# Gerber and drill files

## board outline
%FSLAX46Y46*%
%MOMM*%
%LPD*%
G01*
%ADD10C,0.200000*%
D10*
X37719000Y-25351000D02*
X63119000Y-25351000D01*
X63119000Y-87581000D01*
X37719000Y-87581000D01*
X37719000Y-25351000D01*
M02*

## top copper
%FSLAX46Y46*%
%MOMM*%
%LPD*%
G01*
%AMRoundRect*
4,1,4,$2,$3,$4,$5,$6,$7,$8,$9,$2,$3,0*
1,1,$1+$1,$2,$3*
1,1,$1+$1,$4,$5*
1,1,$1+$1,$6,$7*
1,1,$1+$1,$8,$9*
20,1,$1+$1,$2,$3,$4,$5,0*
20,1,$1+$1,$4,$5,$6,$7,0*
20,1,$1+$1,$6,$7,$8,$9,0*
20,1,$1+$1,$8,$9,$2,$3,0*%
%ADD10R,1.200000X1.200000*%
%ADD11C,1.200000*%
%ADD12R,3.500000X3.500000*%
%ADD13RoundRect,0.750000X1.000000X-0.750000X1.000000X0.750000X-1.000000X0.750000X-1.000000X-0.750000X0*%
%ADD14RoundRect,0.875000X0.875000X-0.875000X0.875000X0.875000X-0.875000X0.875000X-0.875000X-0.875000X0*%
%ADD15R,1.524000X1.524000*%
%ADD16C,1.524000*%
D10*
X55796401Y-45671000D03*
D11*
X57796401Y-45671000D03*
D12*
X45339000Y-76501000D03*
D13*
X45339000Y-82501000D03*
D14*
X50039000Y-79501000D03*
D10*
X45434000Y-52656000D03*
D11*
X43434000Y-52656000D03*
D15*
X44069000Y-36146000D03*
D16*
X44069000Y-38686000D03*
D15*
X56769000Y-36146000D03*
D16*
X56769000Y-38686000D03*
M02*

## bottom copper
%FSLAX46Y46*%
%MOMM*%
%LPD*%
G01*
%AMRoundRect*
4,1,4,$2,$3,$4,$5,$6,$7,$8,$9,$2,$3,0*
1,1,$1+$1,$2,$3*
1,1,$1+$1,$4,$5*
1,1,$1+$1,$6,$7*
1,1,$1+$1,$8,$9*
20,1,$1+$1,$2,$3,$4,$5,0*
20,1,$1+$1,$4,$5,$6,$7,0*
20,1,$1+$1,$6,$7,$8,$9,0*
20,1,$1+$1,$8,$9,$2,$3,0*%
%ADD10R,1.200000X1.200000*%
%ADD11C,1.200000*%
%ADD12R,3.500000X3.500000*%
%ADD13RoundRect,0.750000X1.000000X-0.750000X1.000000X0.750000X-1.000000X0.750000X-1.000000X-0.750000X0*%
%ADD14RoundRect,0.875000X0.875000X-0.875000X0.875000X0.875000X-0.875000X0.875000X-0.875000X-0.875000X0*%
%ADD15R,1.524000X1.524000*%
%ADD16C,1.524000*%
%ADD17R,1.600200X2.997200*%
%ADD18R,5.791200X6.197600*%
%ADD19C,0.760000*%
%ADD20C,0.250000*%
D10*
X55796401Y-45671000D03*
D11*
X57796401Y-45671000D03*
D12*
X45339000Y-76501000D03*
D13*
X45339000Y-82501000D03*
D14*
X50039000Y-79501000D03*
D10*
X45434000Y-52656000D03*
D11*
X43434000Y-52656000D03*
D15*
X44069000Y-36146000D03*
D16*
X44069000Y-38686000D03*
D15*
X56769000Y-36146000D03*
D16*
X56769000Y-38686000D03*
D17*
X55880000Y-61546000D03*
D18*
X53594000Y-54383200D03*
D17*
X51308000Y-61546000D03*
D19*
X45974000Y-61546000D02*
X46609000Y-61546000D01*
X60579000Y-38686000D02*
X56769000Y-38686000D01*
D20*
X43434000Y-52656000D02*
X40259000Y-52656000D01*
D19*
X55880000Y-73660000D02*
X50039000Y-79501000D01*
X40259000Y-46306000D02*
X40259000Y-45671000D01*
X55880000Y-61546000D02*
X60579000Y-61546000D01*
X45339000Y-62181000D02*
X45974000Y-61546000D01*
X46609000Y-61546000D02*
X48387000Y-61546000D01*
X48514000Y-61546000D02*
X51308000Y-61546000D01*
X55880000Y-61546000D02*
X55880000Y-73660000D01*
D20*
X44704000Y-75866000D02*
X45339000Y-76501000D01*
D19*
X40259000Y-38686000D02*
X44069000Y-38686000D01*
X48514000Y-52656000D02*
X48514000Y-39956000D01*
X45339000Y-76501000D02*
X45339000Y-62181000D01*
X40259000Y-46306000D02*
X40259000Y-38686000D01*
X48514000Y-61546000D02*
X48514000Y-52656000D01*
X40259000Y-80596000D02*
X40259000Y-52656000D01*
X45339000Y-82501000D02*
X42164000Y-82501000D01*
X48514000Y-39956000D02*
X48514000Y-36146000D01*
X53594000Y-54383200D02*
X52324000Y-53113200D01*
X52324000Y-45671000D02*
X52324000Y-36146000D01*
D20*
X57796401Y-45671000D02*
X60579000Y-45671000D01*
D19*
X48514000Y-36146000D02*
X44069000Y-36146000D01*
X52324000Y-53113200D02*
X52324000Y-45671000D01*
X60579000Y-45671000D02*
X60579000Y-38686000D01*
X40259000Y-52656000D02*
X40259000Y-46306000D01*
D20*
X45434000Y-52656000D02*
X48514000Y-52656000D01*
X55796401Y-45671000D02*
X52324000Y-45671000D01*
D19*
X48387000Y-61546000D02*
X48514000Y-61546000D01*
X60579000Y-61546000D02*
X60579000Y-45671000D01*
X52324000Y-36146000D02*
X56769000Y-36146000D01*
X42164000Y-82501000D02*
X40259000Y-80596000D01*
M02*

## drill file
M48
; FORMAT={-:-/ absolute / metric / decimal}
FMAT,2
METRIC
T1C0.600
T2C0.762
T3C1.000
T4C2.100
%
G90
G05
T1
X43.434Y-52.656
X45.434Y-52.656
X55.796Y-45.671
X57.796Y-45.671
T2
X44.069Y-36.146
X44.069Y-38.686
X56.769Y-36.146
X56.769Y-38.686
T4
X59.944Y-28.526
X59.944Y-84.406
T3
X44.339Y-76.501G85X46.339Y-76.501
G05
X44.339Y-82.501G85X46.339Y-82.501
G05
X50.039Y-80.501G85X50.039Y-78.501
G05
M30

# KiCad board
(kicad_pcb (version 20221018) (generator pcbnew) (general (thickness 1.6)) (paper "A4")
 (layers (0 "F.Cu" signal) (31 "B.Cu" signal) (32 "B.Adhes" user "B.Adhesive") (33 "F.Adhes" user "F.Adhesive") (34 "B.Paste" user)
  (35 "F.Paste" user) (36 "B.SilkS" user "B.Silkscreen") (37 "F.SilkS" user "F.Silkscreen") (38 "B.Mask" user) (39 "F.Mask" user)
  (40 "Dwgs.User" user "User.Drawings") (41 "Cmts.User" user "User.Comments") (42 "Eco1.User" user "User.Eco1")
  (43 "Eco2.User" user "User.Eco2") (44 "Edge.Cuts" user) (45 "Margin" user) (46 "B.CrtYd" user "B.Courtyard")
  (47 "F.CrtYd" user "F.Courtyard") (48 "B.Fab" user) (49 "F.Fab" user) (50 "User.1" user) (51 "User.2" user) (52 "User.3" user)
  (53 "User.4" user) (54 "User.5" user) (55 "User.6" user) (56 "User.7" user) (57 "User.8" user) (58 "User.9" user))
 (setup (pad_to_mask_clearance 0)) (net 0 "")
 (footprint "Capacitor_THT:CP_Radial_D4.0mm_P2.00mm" (layer "F.Cu") (at 55.796401 45.671)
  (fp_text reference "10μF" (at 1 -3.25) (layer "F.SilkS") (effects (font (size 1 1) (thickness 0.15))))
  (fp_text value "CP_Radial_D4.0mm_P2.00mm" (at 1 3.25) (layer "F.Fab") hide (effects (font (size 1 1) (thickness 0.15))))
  (pad "1" thru_hole rect (at 0 0) (size 1.2 1.2) (drill 0.6) (layers "*.Cu" "*.Mask"))
  (pad "2" thru_hole circle (at 2 0) (size 1.2 1.2) (drill 0.6) (layers "*.Cu" "*.Mask")))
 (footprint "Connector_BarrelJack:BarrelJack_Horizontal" (layer "F.Cu") (at 45.339 76.501 90)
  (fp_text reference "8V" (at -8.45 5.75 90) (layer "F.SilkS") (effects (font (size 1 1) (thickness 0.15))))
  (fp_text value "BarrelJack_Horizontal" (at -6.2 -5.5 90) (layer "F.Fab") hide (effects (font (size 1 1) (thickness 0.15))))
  (pad "1" thru_hole rect (at 0 0 90) (size 3.5 3.5) (drill oval 1 3) (layers "*.Cu" "*.Mask"))
  (pad "2" thru_hole roundrect (at -6 0 90) (size 3 3.5) (drill oval 1 3) (layers "*.Cu" "*.Mask") (roundrect_rratio 0.25))
  (pad "3" thru_hole roundrect (at -3 4.7 90) (size 3.5 3.5) (drill oval 3 1) (layers "*.Cu" "*.Mask") (roundrect_rratio 0.25)))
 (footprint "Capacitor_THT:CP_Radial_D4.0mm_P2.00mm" (layer "F.Cu") (at 45.434 52.656 180)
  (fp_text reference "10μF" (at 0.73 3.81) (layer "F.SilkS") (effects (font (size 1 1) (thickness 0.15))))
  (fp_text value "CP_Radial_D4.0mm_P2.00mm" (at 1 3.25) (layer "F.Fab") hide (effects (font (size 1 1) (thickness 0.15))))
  (pad "1" thru_hole rect (at 0 0 180) (size 1.2 1.2) (drill 0.6) (layers "*.Cu" "*.Mask"))
  (pad "2" thru_hole circle (at 2 0 180) (size 1.2 1.2) (drill 0.6) (layers "*.Cu" "*.Mask")))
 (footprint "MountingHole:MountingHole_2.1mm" (layer "F.Cu") (at 59.944 28.526)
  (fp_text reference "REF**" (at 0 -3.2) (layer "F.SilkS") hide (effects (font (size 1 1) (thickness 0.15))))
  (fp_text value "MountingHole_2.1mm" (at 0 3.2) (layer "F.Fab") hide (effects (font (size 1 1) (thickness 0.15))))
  (pad "" np_thru_hole circle (at 0 0) (size 2.1 2.1) (drill 2.1) (layers "F&B.Cu" "*.Mask")))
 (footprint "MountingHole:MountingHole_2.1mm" (layer "F.Cu") (at 59.944 84.406)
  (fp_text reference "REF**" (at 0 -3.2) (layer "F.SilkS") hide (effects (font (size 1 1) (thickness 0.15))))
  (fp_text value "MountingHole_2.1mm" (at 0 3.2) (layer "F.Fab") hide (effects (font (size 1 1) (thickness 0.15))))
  (pad "" np_thru_hole circle (at 0 0) (size 2.1 2.1) (drill 2.1) (layers "F&B.Cu" "*.Mask")))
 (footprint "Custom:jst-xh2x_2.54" (layer "F.Cu") (at 44.069 37.416)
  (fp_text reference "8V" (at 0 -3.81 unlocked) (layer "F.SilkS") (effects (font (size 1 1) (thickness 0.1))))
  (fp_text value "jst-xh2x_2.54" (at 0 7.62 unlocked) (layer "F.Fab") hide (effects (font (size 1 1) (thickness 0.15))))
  (pad "1" thru_hole rect (at 0 -1.27) (size 1.524 1.524) (drill 0.762) (layers "*.Cu" "*.Mask"))
  (pad "2" thru_hole circle (at 0 1.27) (size 1.524 1.524) (drill 0.762) (layers "*.Cu" "*.Mask")))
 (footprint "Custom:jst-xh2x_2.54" (layer "F.Cu") (at 56.769 37.416)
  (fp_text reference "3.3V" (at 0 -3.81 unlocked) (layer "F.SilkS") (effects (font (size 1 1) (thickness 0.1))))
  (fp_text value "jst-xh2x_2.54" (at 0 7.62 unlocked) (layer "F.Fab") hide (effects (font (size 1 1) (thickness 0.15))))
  (pad "1" thru_hole rect (at 0 -1.27) (size 1.524 1.524) (drill 0.762) (layers "*.Cu" "*.Mask"))
  (pad "2" thru_hole circle (at 0 1.27) (size 1.524 1.524) (drill 0.762) (layers "*.Cu" "*.Mask")))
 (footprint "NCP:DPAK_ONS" (layer "B.Cu") (at 53.594 57.1645 180)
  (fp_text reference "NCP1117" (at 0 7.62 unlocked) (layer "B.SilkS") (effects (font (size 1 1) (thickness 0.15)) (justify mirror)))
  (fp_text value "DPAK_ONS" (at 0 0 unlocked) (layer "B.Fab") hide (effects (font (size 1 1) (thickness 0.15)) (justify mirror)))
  (pad "1" smd rect (at -2.286 -4.3815 180) (size 1.6002 2.9972) (layers "B.Cu" "B.Paste" "B.Mask"))
  (pad "2" smd rect (at 0 2.7813 180) (size 5.7912 6.1976) (layers "B.Cu" "B.Paste" "B.Mask"))
  (pad "3" smd rect (at 2.286 -4.3815 180) (size 1.6002 2.9972) (layers "B.Cu" "B.Paste" "B.Mask")))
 (gr_rect (start 37.719 25.351) (end 63.119 87.581) (stroke (width 0.2) (type default)) (fill none) (layer "Edge.Cuts"))
 (segment (start 45.974 61.546) (end 46.609 61.546) (width 0.76) (layer "B.Cu") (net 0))
 (segment (start 60.579 38.686) (end 56.769 38.686) (width 0.76) (layer "B.Cu") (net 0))
 (segment (start 43.434 52.656) (end 40.259 52.656) (width 0.25) (layer "B.Cu") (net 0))
 (segment (start 55.88 73.66) (end 50.039 79.501) (width 0.76) (layer "B.Cu") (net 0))
 (segment (start 40.259 46.306) (end 40.259 45.671) (width 0.76) (layer "B.Cu") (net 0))
 (segment (start 55.88 61.546) (end 60.579 61.546) (width 0.76) (layer "B.Cu") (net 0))
 (segment (start 45.339 62.181) (end 45.974 61.546) (width 0.76) (layer "B.Cu") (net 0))
 (segment (start 46.609 61.546) (end 48.387 61.546) (width 0.76) (layer "B.Cu") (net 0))
 (segment (start 48.514 61.546) (end 51.308 61.546) (width 0.76) (layer "B.Cu") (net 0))
 (segment (start 55.88 61.546) (end 55.88 73.66) (width 0.76) (layer "B.Cu") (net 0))
 (segment (start 44.704 75.866) (end 45.339 76.501) (width 0.25) (layer "B.Cu") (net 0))
 (segment (start 40.259 38.686) (end 44.069 38.686) (width 0.76) (layer "B.Cu") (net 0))
 (segment (start 48.514 52.656) (end 48.514 39.956) (width 0.76) (layer "B.Cu") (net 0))
 (segment (start 45.339 76.501) (end 45.339 62.181) (width 0.76) (layer "B.Cu") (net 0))
 (segment (start 40.259 46.306) (end 40.259 38.686) (width 0.76) (layer "B.Cu") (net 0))
 (segment (start 48.514 61.546) (end 48.514 52.656) (width 0.76) (layer "B.Cu") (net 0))
 (segment (start 40.259 80.596) (end 40.259 52.656) (width 0.76) (layer "B.Cu") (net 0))
 (segment (start 45.339 82.501) (end 42.164 82.501) (width 0.76) (layer "B.Cu") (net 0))
 (segment (start 48.514 39.956) (end 48.514 36.146) (width 0.76) (layer "B.Cu") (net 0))
 (segment (start 53.594 54.3832) (end 52.324 53.1132) (width 0.76) (layer "B.Cu") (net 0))
 (segment (start 52.324 45.671) (end 52.324 36.146) (width 0.76) (layer "B.Cu") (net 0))
 (segment (start 57.796401 45.671) (end 60.579 45.671) (width 0.25) (layer "B.Cu") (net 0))
 (segment (start 48.514 36.146) (end 44.069 36.146) (width 0.76) (layer "B.Cu") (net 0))
 (segment (start 52.324 53.1132) (end 52.324 45.671) (width 0.76) (layer "B.Cu") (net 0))
 (segment (start 60.579 45.671) (end 60.579 38.686) (width 0.76) (layer "B.Cu") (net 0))
 (segment (start 40.259 52.656) (end 40.259 46.306) (width 0.76) (layer "B.Cu") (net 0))
 (segment (start 45.434 52.656) (end 48.514 52.656) (width 0.25) (layer "B.Cu") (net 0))
 (segment (start 55.796401 45.671) (end 52.324 45.671) (width 0.25) (layer "B.Cu") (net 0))
 (segment (start 48.387 61.546) (end 48.514 61.546) (width 0.76) (layer "B.Cu") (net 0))
 (segment (start 60.579 61.546) (end 60.579 45.671) (width 0.76) (layer "B.Cu") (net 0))
 (segment (start 52.324 36.146) (end 56.769 36.146) (width 0.76) (layer "B.Cu") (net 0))
 (segment (start 42.164 82.501) (end 40.259 80.596) (width 0.76) (layer "B.Cu") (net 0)))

